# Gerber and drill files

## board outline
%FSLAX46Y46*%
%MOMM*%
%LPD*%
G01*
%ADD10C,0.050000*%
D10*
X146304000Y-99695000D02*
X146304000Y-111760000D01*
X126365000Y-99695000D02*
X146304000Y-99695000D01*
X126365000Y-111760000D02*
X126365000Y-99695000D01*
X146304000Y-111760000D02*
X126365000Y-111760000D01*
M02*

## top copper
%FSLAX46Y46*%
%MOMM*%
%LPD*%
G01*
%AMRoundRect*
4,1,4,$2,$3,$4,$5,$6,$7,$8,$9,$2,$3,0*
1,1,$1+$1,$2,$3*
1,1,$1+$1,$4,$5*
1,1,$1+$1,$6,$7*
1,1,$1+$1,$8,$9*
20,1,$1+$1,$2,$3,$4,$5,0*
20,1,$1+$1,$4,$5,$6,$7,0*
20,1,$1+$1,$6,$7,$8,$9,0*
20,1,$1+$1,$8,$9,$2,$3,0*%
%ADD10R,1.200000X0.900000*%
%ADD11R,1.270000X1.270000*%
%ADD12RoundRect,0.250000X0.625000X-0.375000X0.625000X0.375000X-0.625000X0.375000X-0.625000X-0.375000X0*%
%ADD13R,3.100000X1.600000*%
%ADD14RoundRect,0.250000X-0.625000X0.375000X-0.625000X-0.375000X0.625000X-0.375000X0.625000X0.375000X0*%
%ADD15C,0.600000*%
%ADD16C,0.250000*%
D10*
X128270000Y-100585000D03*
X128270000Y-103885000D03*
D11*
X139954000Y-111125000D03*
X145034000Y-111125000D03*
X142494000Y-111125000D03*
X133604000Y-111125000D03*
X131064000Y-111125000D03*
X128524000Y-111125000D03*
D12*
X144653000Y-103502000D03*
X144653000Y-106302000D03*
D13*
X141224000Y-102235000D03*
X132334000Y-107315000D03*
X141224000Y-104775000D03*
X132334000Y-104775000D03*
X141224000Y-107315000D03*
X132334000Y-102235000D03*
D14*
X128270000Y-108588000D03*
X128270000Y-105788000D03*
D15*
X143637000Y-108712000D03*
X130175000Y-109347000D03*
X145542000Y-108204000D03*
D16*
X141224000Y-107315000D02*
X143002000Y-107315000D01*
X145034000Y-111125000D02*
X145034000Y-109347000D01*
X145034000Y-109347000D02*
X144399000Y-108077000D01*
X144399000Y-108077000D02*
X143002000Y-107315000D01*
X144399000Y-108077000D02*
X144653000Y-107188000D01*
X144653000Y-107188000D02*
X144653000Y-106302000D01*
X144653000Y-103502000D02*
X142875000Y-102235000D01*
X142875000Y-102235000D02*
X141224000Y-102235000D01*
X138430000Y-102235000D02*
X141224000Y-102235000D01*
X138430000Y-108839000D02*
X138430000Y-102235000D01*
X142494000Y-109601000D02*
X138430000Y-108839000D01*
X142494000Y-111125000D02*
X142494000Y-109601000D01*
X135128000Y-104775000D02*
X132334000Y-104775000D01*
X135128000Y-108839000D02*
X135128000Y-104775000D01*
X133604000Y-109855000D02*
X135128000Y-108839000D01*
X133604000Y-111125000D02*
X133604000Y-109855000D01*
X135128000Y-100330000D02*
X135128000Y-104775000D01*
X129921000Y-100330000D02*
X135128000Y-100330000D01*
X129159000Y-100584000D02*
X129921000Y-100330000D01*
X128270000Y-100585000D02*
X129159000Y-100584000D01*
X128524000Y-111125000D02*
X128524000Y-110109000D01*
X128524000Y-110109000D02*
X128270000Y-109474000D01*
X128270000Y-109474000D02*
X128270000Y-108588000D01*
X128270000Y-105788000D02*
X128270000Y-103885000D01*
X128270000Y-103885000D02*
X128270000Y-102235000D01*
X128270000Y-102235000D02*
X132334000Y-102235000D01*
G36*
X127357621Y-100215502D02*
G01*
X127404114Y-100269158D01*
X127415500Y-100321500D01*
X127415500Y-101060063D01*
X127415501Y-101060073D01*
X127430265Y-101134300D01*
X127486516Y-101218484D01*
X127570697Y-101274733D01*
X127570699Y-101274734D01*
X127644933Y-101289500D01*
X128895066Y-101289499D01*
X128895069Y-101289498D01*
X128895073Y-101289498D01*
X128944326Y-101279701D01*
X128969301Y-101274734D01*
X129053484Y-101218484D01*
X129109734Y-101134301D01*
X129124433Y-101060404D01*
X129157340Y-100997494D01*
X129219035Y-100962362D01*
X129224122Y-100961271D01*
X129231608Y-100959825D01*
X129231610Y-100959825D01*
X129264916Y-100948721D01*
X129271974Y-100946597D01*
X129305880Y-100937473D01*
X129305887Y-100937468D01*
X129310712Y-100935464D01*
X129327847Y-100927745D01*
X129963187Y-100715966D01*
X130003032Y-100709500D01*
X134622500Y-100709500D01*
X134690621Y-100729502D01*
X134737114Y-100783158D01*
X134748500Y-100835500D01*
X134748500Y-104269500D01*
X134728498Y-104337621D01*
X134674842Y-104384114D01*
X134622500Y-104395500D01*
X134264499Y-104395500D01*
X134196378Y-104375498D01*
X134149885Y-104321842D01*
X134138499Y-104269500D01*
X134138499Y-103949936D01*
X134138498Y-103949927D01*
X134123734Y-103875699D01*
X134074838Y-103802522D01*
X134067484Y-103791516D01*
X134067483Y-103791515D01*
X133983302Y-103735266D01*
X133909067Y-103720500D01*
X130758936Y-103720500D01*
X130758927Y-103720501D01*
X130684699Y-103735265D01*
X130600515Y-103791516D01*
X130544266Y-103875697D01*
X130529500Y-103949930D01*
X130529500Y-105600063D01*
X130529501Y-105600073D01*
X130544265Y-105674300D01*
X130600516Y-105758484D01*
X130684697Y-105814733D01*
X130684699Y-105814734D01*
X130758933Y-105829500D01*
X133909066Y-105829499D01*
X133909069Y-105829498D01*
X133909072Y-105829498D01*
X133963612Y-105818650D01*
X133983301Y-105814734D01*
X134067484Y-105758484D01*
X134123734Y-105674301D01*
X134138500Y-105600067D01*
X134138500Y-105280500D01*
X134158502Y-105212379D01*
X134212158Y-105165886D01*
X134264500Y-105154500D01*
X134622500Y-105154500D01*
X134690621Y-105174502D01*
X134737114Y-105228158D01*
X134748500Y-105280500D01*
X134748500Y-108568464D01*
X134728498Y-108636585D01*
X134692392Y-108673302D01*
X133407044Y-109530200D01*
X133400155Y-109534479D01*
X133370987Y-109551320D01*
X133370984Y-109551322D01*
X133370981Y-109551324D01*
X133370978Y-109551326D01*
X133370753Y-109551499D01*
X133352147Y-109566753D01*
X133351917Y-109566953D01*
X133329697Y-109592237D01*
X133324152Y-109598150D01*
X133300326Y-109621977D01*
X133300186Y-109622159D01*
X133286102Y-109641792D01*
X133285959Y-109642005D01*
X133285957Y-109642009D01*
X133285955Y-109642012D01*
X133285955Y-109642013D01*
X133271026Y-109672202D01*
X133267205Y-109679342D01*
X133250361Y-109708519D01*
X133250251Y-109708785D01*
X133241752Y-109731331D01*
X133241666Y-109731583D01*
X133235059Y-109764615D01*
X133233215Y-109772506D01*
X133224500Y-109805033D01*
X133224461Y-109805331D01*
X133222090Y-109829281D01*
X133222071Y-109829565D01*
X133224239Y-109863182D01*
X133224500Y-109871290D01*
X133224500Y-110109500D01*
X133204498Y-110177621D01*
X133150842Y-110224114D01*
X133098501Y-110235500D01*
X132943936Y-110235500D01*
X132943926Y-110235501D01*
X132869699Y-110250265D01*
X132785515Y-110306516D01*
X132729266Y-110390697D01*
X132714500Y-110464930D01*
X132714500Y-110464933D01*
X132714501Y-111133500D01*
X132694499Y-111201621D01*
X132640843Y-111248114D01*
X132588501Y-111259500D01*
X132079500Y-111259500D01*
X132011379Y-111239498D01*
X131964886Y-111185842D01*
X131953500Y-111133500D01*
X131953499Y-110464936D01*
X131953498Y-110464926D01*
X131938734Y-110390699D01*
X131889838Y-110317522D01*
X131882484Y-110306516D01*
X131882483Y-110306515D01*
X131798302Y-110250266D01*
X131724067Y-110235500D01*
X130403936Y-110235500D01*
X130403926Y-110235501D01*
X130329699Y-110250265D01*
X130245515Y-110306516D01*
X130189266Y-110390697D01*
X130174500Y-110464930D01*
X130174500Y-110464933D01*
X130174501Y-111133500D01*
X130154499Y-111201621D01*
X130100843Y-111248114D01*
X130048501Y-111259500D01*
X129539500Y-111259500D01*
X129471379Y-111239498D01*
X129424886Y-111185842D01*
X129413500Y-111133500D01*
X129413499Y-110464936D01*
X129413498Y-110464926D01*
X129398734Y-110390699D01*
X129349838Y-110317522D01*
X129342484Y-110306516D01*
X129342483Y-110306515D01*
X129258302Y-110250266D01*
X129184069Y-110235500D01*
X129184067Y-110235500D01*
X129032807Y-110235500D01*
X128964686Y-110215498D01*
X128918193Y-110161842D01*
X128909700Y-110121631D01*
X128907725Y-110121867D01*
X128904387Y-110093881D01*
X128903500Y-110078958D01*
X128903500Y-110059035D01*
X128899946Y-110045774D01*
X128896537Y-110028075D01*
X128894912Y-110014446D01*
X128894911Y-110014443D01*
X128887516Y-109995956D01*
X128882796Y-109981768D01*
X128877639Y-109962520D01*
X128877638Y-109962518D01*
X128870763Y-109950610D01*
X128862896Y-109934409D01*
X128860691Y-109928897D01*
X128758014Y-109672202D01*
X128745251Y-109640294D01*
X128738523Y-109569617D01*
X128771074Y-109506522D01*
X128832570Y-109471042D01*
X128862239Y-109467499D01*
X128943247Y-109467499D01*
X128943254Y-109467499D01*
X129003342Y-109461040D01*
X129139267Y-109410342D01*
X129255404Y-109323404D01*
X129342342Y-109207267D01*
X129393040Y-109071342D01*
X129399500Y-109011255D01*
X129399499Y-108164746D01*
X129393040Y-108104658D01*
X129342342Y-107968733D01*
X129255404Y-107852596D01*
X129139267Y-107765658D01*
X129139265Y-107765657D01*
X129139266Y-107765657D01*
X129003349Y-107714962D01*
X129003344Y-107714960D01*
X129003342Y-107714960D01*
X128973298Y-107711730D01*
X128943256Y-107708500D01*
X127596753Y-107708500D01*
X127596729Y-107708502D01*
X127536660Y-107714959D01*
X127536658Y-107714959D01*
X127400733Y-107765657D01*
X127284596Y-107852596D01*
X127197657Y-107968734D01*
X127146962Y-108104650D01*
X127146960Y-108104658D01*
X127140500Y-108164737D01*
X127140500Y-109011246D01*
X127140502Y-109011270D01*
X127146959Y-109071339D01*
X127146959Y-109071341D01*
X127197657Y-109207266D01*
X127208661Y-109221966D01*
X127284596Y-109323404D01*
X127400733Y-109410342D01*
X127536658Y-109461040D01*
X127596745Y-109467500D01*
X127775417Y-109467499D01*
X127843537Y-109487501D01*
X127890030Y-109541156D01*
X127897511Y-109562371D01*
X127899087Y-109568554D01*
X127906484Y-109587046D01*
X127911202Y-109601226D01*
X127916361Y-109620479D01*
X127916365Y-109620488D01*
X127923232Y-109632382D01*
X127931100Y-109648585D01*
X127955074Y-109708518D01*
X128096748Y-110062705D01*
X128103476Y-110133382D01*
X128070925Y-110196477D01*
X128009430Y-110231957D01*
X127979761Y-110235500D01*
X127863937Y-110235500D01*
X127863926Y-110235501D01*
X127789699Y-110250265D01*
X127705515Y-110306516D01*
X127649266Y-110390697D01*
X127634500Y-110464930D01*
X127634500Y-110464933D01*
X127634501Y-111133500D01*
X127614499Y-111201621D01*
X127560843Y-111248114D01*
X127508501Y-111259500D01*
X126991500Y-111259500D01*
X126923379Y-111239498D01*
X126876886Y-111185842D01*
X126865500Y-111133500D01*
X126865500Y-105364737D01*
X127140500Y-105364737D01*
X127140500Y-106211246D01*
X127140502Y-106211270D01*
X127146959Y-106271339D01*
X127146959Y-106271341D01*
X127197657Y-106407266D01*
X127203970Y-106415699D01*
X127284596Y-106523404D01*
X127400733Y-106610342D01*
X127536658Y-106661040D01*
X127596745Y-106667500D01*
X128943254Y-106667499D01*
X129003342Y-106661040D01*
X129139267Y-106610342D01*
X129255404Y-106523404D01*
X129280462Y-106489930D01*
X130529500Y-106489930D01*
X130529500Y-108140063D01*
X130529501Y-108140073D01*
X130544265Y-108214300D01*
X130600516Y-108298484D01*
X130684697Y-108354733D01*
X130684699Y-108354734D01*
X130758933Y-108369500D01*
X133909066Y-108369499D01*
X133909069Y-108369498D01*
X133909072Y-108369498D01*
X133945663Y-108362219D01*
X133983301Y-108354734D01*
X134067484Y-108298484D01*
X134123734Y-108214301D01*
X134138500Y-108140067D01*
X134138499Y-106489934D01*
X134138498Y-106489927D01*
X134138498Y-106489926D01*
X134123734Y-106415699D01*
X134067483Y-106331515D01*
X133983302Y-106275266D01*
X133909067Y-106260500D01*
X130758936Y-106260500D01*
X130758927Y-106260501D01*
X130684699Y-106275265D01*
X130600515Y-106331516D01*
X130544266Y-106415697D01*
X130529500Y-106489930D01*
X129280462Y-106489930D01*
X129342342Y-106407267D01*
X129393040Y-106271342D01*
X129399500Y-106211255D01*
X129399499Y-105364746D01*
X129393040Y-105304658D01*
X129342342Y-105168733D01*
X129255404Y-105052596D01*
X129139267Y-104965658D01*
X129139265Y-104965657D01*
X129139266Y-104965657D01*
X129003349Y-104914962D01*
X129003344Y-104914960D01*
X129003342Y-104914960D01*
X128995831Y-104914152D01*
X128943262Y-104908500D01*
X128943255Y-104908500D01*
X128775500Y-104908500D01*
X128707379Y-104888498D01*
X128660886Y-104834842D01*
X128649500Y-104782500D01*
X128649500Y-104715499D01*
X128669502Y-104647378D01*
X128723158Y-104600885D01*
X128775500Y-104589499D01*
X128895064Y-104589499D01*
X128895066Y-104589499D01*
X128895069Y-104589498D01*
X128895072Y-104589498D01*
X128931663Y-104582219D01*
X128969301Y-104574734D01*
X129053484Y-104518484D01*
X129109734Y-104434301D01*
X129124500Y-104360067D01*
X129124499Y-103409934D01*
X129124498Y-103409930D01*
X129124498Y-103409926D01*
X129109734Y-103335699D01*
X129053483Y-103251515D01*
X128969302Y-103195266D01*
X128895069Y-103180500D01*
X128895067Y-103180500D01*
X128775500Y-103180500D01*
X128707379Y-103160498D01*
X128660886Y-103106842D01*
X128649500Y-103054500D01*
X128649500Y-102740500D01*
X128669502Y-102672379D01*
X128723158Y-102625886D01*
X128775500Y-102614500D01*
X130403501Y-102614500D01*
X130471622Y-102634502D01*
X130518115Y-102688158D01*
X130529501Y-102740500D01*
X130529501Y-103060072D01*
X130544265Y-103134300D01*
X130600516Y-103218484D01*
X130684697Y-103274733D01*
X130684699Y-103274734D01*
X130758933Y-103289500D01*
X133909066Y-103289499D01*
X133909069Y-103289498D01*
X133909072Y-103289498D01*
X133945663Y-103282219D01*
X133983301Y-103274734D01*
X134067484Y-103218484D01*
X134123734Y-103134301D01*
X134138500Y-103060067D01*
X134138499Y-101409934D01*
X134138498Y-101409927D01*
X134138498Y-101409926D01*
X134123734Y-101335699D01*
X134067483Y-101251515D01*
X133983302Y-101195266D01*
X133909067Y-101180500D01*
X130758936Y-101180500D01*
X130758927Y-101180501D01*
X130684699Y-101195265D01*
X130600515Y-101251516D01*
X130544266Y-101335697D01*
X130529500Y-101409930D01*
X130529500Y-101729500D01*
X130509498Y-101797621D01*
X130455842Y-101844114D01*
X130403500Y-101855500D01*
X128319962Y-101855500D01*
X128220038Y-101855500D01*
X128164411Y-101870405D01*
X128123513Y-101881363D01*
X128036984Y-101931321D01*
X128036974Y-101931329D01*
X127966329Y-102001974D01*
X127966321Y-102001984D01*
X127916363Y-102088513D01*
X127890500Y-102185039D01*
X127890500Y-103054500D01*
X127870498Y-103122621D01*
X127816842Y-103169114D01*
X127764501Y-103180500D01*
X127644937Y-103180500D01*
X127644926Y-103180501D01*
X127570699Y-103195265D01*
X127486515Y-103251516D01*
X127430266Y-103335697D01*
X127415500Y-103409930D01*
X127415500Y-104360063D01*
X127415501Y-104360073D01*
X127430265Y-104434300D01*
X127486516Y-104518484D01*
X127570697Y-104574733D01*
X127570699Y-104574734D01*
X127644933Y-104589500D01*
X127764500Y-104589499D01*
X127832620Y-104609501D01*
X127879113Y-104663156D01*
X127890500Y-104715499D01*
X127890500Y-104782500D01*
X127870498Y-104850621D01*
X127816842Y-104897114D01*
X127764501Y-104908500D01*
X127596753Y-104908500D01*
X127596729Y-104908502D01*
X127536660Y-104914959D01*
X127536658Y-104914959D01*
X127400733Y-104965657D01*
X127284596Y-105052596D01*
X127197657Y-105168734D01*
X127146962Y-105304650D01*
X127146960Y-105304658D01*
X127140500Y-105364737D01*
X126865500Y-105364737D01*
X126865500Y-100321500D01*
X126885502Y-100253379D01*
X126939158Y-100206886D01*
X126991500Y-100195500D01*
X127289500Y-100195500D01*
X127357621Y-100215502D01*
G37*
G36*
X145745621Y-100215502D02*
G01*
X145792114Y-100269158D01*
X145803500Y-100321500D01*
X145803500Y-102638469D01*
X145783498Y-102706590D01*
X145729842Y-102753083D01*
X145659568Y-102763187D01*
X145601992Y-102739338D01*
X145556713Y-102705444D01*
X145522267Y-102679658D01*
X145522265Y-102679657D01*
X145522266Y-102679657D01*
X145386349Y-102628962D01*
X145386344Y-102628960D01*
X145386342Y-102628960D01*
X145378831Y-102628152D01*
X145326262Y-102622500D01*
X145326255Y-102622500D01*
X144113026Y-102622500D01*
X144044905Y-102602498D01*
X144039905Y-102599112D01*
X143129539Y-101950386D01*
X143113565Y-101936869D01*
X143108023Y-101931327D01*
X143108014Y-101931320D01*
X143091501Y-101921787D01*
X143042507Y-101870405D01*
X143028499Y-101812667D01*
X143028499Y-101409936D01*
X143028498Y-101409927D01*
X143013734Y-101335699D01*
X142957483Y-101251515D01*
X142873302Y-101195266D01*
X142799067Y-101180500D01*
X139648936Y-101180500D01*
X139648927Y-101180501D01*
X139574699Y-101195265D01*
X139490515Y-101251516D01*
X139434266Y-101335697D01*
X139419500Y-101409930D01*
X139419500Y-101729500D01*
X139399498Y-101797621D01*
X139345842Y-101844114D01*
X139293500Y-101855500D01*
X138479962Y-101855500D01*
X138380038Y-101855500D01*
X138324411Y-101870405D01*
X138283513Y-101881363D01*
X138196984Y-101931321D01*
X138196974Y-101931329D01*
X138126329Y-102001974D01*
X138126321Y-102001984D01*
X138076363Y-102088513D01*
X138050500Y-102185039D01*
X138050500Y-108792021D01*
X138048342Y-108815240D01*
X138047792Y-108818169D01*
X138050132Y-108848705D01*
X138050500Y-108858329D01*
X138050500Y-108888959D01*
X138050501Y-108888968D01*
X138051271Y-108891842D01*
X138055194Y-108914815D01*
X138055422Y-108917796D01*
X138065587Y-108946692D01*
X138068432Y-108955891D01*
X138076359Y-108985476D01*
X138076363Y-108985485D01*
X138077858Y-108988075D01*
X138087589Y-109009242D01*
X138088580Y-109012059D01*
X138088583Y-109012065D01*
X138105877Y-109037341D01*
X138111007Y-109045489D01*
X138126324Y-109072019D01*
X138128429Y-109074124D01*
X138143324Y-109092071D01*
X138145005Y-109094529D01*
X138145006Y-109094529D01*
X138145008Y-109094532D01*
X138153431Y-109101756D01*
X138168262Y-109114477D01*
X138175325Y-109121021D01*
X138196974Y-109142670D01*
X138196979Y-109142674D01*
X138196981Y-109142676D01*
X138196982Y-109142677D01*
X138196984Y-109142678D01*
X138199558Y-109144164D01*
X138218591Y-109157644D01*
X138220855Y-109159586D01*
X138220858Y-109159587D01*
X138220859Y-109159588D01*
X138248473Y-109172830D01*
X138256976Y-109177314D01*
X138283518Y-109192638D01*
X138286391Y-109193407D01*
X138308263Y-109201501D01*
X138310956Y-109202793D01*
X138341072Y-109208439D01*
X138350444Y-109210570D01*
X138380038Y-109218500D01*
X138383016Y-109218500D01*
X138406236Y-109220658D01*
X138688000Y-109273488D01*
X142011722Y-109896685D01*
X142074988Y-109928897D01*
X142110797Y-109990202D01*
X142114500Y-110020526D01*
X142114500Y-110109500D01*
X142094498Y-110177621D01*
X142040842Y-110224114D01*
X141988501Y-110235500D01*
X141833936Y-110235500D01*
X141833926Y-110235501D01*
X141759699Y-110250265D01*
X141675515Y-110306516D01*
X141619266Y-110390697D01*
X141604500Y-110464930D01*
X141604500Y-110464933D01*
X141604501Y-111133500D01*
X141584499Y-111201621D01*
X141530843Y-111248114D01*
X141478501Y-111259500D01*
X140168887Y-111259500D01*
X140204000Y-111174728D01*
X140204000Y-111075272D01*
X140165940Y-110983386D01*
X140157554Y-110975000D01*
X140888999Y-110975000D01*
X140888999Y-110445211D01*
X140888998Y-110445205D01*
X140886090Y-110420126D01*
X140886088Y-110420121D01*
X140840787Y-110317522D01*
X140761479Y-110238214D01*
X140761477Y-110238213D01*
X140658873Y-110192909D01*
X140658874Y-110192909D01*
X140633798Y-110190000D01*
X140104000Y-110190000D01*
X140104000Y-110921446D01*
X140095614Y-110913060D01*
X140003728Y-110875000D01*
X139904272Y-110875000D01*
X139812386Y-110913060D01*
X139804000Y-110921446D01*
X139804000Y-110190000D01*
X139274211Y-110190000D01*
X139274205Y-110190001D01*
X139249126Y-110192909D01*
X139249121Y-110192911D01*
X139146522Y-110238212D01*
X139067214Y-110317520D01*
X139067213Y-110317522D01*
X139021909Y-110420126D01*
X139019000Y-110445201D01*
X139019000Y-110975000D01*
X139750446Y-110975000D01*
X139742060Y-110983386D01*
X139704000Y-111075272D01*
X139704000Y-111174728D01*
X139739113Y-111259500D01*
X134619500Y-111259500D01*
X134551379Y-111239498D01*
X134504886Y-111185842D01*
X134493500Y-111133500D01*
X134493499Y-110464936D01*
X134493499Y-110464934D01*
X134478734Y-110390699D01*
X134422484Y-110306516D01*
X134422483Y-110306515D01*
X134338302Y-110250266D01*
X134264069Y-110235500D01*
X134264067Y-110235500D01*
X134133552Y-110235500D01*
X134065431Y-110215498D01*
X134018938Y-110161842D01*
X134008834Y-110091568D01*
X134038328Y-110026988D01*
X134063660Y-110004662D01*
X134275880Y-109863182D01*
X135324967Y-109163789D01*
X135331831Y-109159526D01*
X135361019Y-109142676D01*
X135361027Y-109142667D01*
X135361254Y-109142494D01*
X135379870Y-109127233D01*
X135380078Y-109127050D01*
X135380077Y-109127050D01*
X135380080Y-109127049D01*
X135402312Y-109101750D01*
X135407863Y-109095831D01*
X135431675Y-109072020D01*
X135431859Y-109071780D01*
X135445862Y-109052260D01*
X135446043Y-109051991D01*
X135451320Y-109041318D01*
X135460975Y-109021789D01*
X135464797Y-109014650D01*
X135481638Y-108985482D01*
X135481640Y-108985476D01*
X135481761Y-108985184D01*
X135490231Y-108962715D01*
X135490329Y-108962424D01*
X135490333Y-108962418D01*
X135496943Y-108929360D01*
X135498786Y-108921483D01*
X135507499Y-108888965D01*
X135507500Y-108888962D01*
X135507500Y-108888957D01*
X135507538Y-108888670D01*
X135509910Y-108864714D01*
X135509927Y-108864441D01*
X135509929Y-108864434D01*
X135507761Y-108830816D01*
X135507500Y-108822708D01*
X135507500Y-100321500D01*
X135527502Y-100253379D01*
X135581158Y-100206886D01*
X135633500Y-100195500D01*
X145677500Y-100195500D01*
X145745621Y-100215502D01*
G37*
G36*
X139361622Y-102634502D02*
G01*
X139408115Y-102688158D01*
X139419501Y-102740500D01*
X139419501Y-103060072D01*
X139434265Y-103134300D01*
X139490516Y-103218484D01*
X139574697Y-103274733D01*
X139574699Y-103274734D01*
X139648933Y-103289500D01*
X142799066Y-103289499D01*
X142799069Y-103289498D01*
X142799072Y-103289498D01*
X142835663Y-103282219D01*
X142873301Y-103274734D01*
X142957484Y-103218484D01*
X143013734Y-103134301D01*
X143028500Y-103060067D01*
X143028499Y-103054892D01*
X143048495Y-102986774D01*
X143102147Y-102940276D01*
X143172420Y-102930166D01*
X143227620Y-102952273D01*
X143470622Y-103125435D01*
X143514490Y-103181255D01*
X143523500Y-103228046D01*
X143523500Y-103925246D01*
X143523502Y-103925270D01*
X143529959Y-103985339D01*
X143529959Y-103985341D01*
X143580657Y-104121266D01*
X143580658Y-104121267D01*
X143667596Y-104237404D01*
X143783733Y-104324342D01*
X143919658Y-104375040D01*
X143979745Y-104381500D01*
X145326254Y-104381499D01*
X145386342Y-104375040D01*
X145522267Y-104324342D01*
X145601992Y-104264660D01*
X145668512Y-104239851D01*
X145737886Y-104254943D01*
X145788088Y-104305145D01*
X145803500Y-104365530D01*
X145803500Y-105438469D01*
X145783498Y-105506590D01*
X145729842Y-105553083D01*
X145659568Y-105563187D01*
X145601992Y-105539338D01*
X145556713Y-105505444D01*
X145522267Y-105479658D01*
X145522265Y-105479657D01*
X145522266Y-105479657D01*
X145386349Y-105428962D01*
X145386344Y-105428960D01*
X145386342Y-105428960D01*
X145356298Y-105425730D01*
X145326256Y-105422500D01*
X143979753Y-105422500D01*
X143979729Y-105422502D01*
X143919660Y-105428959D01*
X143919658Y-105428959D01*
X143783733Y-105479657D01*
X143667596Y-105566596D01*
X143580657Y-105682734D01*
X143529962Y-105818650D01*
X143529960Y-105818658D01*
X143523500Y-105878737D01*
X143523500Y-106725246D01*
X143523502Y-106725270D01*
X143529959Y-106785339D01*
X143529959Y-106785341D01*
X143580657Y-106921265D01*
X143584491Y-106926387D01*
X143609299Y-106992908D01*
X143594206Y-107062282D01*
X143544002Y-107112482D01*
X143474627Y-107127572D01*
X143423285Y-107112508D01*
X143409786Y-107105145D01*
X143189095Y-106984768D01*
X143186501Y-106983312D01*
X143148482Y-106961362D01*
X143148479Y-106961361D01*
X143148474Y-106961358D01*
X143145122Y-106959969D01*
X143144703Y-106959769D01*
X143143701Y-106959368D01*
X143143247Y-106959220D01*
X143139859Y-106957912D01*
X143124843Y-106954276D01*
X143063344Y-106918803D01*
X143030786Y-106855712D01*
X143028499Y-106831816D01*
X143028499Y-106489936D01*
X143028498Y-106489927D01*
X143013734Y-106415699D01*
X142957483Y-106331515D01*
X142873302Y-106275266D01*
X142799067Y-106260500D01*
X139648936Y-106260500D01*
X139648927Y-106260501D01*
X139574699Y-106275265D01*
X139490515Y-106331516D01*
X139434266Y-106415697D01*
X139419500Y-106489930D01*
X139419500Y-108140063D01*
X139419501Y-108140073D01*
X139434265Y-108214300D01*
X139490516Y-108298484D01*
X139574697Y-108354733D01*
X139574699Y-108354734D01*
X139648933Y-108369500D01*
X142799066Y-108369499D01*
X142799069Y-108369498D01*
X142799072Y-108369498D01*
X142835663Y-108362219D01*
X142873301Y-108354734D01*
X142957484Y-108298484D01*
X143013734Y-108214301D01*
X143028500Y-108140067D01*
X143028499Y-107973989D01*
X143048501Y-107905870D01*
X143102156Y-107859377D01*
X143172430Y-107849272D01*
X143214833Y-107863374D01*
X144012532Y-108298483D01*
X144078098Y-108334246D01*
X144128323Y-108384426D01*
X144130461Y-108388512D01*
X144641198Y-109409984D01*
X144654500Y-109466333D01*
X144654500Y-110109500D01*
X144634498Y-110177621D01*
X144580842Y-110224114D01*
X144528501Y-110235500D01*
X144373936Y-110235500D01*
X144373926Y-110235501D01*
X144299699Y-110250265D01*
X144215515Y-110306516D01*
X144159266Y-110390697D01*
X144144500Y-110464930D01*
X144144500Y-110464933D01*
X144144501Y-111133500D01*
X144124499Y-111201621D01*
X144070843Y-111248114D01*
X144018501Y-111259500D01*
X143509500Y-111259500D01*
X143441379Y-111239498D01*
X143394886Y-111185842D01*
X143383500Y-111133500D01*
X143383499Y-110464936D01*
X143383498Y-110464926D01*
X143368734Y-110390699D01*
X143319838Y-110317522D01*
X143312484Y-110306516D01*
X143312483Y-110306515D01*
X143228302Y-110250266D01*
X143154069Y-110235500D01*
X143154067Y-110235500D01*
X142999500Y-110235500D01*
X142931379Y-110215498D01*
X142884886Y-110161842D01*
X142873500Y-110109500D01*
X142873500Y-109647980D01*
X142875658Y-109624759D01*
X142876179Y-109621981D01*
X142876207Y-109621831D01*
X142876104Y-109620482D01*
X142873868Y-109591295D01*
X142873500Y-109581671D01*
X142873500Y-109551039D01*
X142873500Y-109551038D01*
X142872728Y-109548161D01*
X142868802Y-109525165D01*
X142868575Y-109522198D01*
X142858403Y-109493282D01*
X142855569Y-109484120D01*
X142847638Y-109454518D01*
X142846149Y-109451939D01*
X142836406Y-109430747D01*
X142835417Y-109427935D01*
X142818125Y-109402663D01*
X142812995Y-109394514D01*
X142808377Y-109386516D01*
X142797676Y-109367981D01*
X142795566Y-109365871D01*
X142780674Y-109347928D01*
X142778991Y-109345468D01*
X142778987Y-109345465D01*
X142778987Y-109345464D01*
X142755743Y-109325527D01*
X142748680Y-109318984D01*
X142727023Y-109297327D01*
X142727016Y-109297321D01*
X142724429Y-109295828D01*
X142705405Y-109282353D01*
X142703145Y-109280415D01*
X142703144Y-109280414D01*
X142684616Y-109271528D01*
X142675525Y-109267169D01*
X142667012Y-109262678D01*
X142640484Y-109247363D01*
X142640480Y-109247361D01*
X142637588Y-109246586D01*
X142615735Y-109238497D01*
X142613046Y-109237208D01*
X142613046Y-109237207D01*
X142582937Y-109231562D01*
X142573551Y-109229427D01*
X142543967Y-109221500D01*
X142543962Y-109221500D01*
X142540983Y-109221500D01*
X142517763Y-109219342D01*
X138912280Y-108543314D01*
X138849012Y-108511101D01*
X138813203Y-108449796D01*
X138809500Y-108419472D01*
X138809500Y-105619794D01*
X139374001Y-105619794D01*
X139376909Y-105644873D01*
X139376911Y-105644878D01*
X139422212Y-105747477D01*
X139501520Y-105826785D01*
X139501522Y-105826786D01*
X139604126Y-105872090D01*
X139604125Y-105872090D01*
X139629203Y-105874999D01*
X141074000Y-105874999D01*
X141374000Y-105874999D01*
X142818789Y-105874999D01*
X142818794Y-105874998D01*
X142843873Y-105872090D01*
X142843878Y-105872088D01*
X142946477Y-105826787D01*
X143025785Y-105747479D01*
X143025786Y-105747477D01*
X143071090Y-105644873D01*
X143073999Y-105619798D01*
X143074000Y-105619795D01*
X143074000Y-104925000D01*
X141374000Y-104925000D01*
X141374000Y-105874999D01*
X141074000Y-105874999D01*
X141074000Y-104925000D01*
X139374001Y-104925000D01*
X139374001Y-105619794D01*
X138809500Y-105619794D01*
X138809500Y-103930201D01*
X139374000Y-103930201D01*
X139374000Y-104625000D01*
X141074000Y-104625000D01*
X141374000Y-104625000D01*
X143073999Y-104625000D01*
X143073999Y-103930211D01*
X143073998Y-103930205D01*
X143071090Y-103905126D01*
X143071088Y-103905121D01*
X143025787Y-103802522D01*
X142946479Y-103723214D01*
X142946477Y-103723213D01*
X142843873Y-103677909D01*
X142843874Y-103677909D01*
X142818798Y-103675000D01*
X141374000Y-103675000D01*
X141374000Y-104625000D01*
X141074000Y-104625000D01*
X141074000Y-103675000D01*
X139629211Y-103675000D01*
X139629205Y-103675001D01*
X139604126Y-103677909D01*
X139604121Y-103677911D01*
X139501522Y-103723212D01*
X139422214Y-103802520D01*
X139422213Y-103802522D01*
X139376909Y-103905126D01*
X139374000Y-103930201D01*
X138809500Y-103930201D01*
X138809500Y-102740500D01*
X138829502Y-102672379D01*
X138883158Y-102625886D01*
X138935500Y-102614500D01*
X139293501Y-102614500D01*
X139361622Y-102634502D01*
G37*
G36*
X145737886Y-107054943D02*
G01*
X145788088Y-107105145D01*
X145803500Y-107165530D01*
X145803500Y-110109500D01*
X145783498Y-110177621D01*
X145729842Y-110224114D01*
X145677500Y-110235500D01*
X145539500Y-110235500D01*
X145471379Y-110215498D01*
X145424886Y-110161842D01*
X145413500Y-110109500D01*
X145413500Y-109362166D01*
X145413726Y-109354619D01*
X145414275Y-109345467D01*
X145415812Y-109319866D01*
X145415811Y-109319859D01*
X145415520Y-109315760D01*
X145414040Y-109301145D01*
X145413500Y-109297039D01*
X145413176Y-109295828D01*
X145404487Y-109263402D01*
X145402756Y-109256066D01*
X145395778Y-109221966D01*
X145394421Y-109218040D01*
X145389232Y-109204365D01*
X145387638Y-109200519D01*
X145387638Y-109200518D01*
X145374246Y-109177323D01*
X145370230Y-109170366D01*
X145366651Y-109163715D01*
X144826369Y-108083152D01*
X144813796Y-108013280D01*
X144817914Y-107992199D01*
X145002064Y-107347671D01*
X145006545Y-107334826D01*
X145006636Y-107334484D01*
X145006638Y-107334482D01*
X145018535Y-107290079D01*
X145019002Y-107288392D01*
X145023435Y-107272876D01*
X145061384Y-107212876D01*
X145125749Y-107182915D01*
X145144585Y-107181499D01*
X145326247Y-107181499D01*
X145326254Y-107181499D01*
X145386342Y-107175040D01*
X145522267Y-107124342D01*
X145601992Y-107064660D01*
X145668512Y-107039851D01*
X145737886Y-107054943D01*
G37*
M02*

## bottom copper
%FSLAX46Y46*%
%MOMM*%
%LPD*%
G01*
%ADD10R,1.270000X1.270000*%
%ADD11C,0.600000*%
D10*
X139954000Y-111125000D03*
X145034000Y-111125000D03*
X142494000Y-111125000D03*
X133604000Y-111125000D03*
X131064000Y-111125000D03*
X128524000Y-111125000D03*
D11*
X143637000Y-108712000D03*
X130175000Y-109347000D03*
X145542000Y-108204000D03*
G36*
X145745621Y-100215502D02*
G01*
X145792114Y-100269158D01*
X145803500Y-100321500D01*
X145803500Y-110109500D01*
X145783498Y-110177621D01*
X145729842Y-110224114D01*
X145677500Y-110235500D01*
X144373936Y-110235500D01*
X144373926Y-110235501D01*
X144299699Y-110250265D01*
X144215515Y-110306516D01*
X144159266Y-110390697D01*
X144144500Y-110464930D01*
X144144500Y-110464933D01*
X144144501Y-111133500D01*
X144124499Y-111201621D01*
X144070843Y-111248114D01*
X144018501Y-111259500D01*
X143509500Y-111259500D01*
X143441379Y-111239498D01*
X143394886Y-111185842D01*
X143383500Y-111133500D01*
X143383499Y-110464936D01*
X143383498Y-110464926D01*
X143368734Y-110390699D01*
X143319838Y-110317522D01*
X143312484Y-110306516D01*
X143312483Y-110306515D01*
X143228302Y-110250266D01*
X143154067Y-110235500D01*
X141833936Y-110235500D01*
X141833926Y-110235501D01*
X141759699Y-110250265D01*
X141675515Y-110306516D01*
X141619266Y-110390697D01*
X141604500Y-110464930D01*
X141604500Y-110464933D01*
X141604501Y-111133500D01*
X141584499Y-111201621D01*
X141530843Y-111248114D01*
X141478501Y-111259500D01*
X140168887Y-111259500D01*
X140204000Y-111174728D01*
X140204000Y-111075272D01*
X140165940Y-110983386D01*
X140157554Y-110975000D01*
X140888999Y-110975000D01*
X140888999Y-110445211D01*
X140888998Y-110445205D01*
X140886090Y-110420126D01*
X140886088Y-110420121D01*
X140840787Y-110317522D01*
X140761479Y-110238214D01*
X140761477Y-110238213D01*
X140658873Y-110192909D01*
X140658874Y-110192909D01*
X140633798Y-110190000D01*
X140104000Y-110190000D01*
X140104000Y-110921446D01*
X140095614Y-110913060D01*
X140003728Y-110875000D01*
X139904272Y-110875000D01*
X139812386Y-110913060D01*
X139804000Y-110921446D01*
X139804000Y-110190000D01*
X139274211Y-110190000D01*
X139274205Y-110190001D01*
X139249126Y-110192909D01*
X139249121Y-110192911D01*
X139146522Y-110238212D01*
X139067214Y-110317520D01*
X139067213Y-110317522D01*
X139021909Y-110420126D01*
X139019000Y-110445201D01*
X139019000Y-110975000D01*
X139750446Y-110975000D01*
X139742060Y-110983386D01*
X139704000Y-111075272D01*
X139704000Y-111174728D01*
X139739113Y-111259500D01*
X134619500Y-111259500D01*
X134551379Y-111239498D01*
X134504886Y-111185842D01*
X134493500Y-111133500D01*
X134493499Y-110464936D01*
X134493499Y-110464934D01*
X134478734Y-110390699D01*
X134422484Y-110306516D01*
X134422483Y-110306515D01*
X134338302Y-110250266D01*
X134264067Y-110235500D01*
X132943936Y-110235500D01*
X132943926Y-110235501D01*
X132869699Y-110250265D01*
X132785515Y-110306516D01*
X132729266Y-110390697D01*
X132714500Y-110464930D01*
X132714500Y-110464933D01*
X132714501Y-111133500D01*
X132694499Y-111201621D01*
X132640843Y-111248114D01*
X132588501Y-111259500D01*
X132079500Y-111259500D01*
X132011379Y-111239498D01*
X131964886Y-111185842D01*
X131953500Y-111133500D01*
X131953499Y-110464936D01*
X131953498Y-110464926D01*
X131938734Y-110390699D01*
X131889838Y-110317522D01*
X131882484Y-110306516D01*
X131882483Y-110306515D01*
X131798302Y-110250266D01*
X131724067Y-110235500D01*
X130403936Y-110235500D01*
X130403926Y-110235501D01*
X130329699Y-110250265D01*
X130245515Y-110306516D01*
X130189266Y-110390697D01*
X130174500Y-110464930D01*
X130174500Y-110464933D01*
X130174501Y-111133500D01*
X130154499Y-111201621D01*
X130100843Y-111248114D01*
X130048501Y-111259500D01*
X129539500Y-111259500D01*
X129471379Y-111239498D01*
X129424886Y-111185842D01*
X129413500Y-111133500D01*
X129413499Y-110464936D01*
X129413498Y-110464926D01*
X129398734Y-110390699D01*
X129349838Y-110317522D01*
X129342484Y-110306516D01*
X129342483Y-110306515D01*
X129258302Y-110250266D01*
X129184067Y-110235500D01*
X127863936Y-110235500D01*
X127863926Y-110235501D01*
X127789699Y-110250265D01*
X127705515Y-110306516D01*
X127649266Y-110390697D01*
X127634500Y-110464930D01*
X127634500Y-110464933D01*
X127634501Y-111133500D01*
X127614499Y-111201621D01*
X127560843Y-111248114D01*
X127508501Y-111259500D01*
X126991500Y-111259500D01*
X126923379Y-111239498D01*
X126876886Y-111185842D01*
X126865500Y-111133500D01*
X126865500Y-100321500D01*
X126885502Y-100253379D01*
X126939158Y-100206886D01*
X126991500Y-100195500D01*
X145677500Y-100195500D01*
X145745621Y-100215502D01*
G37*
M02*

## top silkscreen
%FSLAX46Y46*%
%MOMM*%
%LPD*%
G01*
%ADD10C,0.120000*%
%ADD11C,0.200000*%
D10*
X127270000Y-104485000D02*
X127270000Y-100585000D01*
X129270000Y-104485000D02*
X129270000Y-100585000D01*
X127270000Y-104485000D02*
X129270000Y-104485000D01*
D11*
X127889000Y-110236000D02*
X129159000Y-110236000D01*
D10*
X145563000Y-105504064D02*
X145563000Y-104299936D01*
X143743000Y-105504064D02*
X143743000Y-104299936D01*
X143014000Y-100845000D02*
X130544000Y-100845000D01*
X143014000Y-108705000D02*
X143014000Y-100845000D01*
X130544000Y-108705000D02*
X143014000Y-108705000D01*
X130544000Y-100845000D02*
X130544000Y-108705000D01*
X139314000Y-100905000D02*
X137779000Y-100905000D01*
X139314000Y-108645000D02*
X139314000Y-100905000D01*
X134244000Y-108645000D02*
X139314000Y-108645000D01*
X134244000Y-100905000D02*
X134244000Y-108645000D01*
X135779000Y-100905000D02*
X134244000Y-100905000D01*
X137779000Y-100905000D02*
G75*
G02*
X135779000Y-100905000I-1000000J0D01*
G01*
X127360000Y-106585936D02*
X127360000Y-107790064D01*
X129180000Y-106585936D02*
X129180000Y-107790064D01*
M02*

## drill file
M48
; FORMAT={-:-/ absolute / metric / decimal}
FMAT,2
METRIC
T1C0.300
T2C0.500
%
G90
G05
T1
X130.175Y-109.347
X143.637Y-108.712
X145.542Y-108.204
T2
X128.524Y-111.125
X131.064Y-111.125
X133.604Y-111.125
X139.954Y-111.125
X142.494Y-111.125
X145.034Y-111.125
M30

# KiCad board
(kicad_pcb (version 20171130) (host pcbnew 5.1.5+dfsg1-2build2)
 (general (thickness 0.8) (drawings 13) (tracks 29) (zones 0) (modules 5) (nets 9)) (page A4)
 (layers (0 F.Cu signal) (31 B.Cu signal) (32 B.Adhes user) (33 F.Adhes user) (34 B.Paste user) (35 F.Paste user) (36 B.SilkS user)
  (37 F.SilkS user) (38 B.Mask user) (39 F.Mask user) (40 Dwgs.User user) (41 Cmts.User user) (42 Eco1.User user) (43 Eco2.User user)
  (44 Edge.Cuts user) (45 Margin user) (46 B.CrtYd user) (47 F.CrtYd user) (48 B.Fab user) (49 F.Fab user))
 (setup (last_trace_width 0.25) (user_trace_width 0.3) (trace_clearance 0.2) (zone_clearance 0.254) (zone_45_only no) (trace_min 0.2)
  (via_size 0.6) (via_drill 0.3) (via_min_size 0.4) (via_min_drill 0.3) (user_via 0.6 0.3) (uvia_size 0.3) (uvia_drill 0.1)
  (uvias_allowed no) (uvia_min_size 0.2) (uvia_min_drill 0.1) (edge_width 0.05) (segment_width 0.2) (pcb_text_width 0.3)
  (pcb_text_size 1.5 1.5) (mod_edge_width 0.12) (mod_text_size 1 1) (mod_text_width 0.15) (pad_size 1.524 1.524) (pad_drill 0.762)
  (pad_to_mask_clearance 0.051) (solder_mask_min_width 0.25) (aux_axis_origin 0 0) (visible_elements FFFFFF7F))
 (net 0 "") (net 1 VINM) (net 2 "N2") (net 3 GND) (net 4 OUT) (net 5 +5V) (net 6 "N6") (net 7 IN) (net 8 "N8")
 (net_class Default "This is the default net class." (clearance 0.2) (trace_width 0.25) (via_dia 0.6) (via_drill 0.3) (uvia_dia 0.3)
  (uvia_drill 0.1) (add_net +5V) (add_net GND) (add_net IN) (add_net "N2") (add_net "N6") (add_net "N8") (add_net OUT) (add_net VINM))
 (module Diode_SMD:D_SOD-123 (layer F.Cu) (at 128.27 102.235 90)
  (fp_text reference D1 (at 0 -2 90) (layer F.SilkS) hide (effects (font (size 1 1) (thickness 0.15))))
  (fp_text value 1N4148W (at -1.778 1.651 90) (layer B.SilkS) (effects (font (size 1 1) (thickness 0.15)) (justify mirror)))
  (fp_line (start -2.25 -1) (end 1.65 -1) (layer F.SilkS) (width 0.12))
  (fp_line (start -2.25 1) (end 1.65 1) (layer F.SilkS) (width 0.12))
  (fp_line (start -2.25 -1) (end -2.25 1) (layer F.SilkS) (width 0.12))
  (pad 2 smd rect (at 1.65 0 90) (size 0.9 1.2) (layers F.Cu F.Paste F.Mask) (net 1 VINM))
  (pad 1 smd rect (at -1.65 0 90) (size 0.9 1.2) (layers F.Cu F.Paste F.Mask) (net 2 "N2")))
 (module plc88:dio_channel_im (layer F.Cu) (at 135.509 108.585)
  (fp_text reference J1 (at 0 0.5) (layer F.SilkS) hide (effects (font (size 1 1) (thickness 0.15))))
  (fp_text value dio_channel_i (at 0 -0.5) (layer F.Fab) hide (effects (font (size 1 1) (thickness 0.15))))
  (fp_line (start -7.62 1.651) (end -6.35 1.651) (layer F.SilkS) (width 0.2))
  (pad 4 thru_hole rect (at 4.445 2.54) (size 1.27 1.27) (drill 0.5) (layers *.Cu *.Mask) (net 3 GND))
  (pad 6 thru_hole rect (at 9.525 2.54) (size 1.27 1.27) (drill 0.5) (layers *.Cu *.Mask) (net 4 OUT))
  (pad 5 thru_hole rect (at 6.985 2.54) (size 1.27 1.27) (drill 0.5) (layers *.Cu *.Mask) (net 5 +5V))
  (pad 3 thru_hole rect (at -1.905 2.54) (size 1.27 1.27) (drill 0.5) (layers *.Cu *.Mask) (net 1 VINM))
  (pad 2 thru_hole rect (at -4.445 2.54) (size 1.27 1.27) (drill 0.5) (layers *.Cu *.Mask) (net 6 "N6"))
  (pad 1 thru_hole rect (at -6.985 2.54) (size 1.27 1.27) (drill 0.5) (layers *.Cu *.Mask) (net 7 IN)))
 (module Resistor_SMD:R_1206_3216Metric (layer F.Cu) (at 144.653 104.902 90)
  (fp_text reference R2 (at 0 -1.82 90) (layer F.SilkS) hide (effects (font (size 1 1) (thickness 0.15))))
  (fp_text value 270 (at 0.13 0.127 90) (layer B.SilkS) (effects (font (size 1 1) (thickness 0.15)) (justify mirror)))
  (fp_line (start -0.602064 0.91) (end 0.602064 0.91) (layer F.SilkS) (width 0.12))
  (fp_line (start -0.602064 -0.91) (end 0.602064 -0.91) (layer F.SilkS) (width 0.12))
  (pad 2 smd roundrect (at 1.4 0 90) (size 1.25 1.75) (layers F.Cu F.Paste F.Mask) (roundrect_rratio 0.2) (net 5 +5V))
  (pad 1 smd roundrect (at -1.4 0 90) (size 1.25 1.75) (layers F.Cu F.Paste F.Mask) (roundrect_rratio 0.2) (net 4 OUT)))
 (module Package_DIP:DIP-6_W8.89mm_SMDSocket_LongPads (layer F.Cu) (at 136.779 104.775)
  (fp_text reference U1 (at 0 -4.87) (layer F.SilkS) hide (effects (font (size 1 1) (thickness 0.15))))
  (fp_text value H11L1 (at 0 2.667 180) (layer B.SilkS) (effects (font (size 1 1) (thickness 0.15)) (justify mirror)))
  (fp_line (start 6.235 -3.93) (end -6.235 -3.93) (layer F.SilkS) (width 0.12))
  (fp_line (start 6.235 3.93) (end 6.235 -3.93) (layer F.SilkS) (width 0.12))
  (fp_line (start -6.235 3.93) (end 6.235 3.93) (layer F.SilkS) (width 0.12))
  (fp_line (start -6.235 -3.93) (end -6.235 3.93) (layer F.SilkS) (width 0.12))
  (fp_line (start 2.535 -3.87) (end 1 -3.87) (layer F.SilkS) (width 0.12))
  (fp_line (start 2.535 3.87) (end 2.535 -3.87) (layer F.SilkS) (width 0.12))
  (fp_line (start -2.535 3.87) (end 2.535 3.87) (layer F.SilkS) (width 0.12))
  (fp_line (start -2.535 -3.87) (end -2.535 3.87) (layer F.SilkS) (width 0.12))
  (fp_line (start -1 -3.87) (end -2.535 -3.87) (layer F.SilkS) (width 0.12))
  (fp_arc (start 0 -3.87) (end -1 -3.87) (angle -180) (layer F.SilkS) (width 0.12))
  (pad 6 smd rect (at 4.445 -2.54) (size 3.1 1.6) (layers F.Cu F.Paste F.Mask) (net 5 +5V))
  (pad 3 smd rect (at -4.445 2.54) (size 3.1 1.6) (layers F.Cu F.Paste F.Mask) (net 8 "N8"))
  (pad 5 smd rect (at 4.445 0) (size 3.1 1.6) (layers F.Cu F.Paste F.Mask) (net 3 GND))
  (pad 2 smd rect (at -4.445 0) (size 3.1 1.6) (layers F.Cu F.Paste F.Mask) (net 1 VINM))
  (pad 4 smd rect (at 4.445 2.54) (size 3.1 1.6) (layers F.Cu F.Paste F.Mask) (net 4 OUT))
  (pad 1 smd rect (at -4.445 -2.54) (size 3.1 1.6) (layers F.Cu F.Paste F.Mask) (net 2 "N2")))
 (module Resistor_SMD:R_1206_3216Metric (layer F.Cu) (at 128.27 107.188 270)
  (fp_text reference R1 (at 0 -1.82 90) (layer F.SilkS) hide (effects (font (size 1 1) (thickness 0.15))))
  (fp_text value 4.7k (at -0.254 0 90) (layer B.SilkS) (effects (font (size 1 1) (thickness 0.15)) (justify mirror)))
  (fp_line (start -0.602064 0.91) (end 0.602064 0.91) (layer F.SilkS) (width 0.12))
  (fp_line (start -0.602064 -0.91) (end 0.602064 -0.91) (layer F.SilkS) (width 0.12))
  (pad 2 smd roundrect (at 1.4 0 270) (size 1.25 1.75) (layers F.Cu F.Paste F.Mask) (roundrect_rratio 0.2) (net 7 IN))
  (pad 1 smd roundrect (at -1.4 0 270) (size 1.25 1.75) (layers F.Cu F.Paste F.Mask) (roundrect_rratio 0.2) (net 2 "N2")))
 (gr_line (start 146.304 99.695) (end 146.304 111.76) (layer Edge.Cuts) (width 0.05))
 (gr_line (start 126.365 99.695) (end 146.304 99.695) (layer Edge.Cuts) (width 0.05))
 (gr_line (start 126.365 111.76) (end 126.365 99.695) (layer Edge.Cuts) (width 0.05))
 (gr_line (start 146.304 111.76) (end 126.365 111.76) (layer Edge.Cuts) (width 0.05))
 (segment (start 141.224 107.315) (end 143.002 107.315) (width 0.25) (layer F.Cu) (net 4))
 (segment (start 145.034 111.125) (end 145.034 109.347) (width 0.25) (layer F.Cu) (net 4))
 (segment (start 145.034 109.347) (end 144.399 108.077) (width 0.25) (layer F.Cu) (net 4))
 (segment (start 144.399 108.077) (end 143.002 107.315) (width 0.25) (layer F.Cu) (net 4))
 (segment (start 144.399 108.077) (end 144.653 107.188) (width 0.25) (layer F.Cu) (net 4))
 (segment (start 144.653 107.188) (end 144.653 106.302) (width 0.25) (layer F.Cu) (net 4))
 (segment (start 144.653 103.502) (end 142.875 102.235) (width 0.25) (layer F.Cu) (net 5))
 (segment (start 142.875 102.235) (end 141.224 102.235) (width 0.25) (layer F.Cu) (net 5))
 (segment (start 138.43 102.235) (end 141.224 102.235) (width 0.25) (layer F.Cu) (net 5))
 (segment (start 138.43 108.839) (end 138.43 102.235) (width 0.25) (layer F.Cu) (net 5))
 (segment (start 142.494 109.601) (end 138.43 108.839) (width 0.25) (layer F.Cu) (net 5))
 (segment (start 142.494 111.125) (end 142.494 109.601) (width 0.25) (layer F.Cu) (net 5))
 (via (at 143.637 108.712) (size 0.6) (drill 0.3) (layers F.Cu B.Cu) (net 3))
 (via (at 130.175 109.347) (size 0.6) (drill 0.3) (layers F.Cu B.Cu) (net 3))
 (via (at 145.542 108.204) (size 0.6) (drill 0.3) (layers F.Cu B.Cu) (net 3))
 (segment (start 135.128 104.775) (end 132.334 104.775) (width 0.25) (layer F.Cu) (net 1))
 (segment (start 135.128 108.839) (end 135.128 104.775) (width 0.25) (layer F.Cu) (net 1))
 (segment (start 133.604 109.855) (end 135.128 108.839) (width 0.25) (layer F.Cu) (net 1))
 (segment (start 133.604 111.125) (end 133.604 109.855) (width 0.25) (layer F.Cu) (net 1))
 (segment (start 135.128 100.33) (end 135.128 104.775) (width 0.25) (layer F.Cu) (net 1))
 (segment (start 129.921 100.33) (end 135.128 100.33) (width 0.25) (layer F.Cu) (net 1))
 (segment (start 129.159 100.584) (end 129.921 100.33) (width 0.25) (layer F.Cu) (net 1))
 (segment (start 128.27 100.585) (end 129.159 100.584) (width 0.25) (layer F.Cu) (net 1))
 (segment (start 128.524 111.125) (end 128.524 110.109) (width 0.25) (layer F.Cu) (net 7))
 (segment (start 128.524 110.109) (end 128.27 109.474) (width 0.25) (layer F.Cu) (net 7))
 (segment (start 128.27 109.474) (end 128.27 108.588) (width 0.25) (layer F.Cu) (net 7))
 (segment (start 128.27 105.788) (end 128.27 103.885) (width 0.25) (layer F.Cu) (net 2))
 (segment (start 128.27 103.885) (end 128.27 102.235) (width 0.25) (layer F.Cu) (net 2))
 (segment (start 128.27 102.235) (end 132.334 102.235) (width 0.25) (layer F.Cu) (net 2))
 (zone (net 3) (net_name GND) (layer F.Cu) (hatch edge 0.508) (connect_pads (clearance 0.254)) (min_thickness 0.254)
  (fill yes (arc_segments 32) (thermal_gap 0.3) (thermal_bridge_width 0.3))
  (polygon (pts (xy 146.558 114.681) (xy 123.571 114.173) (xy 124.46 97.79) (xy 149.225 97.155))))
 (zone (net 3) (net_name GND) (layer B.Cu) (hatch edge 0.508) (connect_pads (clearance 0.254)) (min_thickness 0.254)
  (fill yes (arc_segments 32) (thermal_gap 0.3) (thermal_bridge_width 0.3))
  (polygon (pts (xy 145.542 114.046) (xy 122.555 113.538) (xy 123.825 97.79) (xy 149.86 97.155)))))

